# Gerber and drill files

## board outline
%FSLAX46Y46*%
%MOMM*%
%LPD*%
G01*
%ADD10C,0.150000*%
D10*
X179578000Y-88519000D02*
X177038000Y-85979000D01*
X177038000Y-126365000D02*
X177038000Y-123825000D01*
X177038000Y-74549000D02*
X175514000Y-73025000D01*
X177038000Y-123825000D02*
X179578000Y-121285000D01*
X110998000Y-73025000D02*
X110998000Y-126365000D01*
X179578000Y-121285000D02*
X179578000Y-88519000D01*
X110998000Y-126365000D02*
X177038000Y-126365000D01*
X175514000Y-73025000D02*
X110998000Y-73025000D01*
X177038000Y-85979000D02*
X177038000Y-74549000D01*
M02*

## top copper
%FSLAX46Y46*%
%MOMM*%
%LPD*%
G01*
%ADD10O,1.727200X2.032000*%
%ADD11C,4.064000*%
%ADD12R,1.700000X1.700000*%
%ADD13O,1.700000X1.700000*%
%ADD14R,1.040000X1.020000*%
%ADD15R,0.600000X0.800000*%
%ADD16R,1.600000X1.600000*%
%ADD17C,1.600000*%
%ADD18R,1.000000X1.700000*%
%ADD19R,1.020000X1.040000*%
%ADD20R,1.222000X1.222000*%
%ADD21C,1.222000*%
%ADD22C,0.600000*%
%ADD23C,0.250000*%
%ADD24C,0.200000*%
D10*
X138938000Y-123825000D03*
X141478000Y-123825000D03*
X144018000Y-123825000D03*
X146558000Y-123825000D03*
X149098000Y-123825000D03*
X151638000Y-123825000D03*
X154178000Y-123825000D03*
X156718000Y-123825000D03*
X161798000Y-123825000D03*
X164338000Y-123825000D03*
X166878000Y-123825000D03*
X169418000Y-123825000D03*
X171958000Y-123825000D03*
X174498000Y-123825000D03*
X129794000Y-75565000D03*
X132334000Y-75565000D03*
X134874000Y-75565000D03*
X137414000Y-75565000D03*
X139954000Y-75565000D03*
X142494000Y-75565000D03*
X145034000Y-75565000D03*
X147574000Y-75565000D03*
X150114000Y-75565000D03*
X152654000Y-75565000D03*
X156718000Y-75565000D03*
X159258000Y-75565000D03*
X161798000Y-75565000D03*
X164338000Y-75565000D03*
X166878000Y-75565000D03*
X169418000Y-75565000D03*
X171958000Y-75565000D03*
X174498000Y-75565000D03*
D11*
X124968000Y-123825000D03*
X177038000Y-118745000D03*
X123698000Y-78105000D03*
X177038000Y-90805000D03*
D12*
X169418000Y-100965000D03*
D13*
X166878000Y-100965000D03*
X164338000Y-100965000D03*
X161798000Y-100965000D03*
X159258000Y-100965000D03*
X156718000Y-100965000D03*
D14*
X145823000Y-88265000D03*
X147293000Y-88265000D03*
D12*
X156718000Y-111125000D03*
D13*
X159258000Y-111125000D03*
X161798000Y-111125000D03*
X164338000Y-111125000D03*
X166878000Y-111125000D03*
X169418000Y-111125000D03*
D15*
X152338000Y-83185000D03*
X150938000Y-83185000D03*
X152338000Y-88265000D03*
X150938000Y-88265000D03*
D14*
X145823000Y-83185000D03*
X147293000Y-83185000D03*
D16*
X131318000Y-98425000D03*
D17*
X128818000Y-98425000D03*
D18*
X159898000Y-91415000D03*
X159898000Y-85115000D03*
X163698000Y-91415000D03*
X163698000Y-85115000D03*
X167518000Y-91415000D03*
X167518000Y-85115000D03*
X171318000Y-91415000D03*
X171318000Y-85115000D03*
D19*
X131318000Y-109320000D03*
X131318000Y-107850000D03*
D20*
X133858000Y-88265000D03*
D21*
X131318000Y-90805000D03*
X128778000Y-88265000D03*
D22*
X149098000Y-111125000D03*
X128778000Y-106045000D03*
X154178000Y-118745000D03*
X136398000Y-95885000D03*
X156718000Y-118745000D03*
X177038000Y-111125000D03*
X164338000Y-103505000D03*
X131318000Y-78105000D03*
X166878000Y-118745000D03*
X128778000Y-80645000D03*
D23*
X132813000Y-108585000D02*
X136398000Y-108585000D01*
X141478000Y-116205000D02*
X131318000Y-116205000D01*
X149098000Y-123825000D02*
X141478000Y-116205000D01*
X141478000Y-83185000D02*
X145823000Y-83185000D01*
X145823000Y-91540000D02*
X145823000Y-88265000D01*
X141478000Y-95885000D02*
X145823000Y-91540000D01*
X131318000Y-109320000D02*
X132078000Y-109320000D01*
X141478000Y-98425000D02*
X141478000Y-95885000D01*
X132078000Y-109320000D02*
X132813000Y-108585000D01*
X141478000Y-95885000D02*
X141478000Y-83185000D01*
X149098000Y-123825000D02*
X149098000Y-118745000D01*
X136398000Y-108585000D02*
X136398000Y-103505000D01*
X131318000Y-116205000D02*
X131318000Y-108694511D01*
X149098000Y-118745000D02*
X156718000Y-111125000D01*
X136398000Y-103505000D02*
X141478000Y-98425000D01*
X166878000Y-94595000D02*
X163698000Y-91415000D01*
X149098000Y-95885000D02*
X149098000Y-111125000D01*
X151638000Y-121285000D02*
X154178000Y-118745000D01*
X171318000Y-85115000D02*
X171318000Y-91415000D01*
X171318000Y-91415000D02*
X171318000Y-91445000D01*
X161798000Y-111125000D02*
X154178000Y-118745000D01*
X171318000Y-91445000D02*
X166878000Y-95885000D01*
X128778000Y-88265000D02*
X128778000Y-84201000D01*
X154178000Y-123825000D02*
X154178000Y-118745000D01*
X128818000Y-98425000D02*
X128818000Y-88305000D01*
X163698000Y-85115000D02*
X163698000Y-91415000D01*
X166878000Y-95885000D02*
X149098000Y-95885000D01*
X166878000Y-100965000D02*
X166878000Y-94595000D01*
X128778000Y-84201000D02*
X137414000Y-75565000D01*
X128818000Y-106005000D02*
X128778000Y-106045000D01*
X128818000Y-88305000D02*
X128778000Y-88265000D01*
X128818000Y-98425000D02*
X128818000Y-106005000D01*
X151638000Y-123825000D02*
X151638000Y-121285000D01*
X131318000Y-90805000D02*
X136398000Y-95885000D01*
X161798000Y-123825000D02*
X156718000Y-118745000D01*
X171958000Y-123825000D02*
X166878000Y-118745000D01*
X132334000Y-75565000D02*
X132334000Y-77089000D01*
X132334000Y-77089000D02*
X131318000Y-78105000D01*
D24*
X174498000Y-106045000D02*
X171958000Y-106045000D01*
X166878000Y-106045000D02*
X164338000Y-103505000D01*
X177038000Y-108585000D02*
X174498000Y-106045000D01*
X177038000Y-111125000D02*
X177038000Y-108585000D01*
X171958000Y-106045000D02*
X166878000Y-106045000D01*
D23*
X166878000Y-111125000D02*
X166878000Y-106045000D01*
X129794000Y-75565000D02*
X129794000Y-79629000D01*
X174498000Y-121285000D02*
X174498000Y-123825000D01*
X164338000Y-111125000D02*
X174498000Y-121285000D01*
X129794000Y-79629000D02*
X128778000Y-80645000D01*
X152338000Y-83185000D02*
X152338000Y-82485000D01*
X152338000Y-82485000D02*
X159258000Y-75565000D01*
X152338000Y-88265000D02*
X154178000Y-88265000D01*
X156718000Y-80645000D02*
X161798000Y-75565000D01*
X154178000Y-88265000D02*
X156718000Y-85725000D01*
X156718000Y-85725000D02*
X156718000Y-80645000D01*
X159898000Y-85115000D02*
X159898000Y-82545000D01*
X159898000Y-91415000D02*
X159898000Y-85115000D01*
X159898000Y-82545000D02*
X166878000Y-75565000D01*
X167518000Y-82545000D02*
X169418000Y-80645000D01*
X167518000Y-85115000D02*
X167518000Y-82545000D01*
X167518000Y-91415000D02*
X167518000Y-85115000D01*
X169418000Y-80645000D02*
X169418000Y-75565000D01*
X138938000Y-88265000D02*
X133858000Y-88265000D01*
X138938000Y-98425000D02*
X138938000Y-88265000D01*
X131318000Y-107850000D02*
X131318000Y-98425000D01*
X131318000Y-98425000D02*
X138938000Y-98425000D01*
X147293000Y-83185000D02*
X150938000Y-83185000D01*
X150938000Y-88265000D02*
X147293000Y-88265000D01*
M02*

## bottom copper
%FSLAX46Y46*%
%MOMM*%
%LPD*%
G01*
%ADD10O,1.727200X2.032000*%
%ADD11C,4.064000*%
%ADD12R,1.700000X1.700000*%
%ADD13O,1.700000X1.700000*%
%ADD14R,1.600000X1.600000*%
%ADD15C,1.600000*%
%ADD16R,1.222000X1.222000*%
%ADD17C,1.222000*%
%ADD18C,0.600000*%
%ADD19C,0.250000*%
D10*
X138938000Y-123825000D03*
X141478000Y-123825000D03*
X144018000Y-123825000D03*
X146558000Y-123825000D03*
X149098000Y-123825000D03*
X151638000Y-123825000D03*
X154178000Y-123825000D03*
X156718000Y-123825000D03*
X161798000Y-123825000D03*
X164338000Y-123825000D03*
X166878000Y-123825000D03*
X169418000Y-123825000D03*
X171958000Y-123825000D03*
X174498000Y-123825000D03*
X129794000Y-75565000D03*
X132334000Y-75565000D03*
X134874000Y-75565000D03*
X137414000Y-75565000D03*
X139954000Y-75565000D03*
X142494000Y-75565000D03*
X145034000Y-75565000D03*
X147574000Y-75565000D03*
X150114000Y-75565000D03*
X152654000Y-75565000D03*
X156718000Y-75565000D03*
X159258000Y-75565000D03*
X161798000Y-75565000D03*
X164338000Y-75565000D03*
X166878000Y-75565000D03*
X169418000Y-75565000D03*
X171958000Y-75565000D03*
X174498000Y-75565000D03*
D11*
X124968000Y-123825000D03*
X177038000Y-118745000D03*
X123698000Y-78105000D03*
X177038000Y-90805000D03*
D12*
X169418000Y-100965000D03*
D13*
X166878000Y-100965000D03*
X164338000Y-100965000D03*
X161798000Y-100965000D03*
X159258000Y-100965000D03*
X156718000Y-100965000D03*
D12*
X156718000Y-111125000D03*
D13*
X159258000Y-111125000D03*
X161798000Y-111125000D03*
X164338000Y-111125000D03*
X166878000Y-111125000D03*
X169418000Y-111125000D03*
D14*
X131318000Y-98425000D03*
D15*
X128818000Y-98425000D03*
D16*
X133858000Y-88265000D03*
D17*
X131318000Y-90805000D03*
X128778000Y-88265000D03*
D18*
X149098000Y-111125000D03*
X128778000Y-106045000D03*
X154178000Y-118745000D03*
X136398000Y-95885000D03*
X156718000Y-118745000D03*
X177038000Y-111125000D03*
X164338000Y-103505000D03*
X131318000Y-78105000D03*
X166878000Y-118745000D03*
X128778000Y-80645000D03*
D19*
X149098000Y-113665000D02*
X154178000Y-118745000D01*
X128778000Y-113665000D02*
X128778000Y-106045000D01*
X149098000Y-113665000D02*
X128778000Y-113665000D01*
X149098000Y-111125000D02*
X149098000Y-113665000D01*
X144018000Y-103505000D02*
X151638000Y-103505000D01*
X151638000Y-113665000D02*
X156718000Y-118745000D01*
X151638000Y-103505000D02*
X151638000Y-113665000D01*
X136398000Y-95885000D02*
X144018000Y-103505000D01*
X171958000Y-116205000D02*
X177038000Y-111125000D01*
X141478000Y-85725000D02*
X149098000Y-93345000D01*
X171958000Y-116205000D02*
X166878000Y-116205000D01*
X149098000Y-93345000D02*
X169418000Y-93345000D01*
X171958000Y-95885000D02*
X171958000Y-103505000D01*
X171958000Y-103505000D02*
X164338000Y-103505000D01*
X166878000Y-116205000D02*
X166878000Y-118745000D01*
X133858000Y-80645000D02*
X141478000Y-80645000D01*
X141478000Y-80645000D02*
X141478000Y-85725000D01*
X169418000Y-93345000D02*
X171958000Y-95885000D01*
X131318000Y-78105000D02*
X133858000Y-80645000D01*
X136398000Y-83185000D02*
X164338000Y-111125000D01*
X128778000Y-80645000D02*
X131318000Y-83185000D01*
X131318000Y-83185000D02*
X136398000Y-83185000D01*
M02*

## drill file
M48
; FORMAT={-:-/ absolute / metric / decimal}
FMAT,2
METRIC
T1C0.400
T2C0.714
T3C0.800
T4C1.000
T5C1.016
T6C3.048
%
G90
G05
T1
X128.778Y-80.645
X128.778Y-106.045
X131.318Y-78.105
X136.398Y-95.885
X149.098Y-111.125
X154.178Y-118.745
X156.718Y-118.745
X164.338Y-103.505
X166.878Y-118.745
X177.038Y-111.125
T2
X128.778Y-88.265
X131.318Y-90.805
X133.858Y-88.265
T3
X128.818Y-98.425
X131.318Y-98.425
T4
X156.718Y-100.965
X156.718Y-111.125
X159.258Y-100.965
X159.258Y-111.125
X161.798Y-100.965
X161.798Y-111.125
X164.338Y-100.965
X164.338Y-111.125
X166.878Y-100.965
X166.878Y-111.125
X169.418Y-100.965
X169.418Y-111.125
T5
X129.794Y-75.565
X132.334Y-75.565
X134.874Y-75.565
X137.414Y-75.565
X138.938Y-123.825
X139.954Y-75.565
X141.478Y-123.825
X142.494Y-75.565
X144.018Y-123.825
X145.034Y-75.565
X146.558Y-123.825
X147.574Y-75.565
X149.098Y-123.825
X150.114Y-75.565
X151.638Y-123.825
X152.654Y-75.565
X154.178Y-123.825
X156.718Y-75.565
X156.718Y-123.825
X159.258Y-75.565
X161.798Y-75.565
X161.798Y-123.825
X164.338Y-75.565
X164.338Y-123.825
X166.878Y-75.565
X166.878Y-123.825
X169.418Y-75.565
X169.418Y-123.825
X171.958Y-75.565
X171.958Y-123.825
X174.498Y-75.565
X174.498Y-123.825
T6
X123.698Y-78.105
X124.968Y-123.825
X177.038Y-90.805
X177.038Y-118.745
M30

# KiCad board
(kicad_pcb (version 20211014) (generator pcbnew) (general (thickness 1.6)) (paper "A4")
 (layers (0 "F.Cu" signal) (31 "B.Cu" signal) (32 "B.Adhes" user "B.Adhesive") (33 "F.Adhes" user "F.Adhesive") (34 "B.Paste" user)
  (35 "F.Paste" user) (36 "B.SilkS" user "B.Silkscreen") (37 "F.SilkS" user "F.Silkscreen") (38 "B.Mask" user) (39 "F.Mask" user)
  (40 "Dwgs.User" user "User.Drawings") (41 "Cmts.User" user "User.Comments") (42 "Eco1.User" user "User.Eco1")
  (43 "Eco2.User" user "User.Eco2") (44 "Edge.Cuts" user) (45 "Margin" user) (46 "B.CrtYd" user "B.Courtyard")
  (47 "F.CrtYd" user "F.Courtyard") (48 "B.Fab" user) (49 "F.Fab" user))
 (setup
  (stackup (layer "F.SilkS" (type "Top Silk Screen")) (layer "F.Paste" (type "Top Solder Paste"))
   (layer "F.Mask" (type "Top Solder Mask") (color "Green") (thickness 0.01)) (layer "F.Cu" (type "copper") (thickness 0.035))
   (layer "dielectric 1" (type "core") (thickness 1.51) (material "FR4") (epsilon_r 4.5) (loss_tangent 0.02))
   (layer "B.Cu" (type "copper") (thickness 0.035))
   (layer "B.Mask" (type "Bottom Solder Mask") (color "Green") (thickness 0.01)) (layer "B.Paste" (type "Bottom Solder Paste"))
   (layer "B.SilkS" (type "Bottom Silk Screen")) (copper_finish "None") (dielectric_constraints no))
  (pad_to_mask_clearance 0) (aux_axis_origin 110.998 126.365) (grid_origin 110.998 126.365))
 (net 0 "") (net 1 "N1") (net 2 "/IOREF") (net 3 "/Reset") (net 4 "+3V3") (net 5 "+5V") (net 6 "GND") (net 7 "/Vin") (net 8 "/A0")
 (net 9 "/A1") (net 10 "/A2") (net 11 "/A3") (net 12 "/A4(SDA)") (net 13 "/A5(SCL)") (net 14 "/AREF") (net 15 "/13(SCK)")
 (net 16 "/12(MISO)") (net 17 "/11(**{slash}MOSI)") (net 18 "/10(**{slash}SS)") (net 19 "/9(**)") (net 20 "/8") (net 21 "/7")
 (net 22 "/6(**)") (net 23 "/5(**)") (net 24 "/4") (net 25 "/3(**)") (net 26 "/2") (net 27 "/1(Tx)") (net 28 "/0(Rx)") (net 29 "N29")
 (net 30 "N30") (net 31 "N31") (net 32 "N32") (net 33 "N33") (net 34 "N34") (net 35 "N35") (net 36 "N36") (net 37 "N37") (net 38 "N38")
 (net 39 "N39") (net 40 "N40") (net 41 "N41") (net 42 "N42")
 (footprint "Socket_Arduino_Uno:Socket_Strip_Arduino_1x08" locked (layer "F.Cu") (at 138.938 123.825)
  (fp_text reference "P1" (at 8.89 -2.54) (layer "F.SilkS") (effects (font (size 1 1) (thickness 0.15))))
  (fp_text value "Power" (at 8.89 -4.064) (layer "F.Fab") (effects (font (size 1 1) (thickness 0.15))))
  (pad "1" thru_hole oval locked (at 0 0) (size 1.7272 2.032) (drill 1.016) (layers *.Cu *.Mask "F.SilkS") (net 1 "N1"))
  (pad "2" thru_hole oval locked (at 2.54 0) (size 1.7272 2.032) (drill 1.016) (layers *.Cu *.Mask "F.SilkS") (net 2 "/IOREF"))
  (pad "3" thru_hole oval locked (at 5.08 0) (size 1.7272 2.032) (drill 1.016) (layers *.Cu *.Mask "F.SilkS") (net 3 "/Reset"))
  (pad "4" thru_hole oval locked (at 7.62 0) (size 1.7272 2.032) (drill 1.016) (layers *.Cu *.Mask "F.SilkS") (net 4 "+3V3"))
  (pad "5" thru_hole oval locked (at 10.16 0) (size 1.7272 2.032) (drill 1.016) (layers *.Cu *.Mask "F.SilkS") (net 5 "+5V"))
  (pad "6" thru_hole oval locked (at 12.7 0) (size 1.7272 2.032) (drill 1.016) (layers *.Cu *.Mask "F.SilkS") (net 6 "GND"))
  (pad "7" thru_hole oval locked (at 15.24 0) (size 1.7272 2.032) (drill 1.016) (layers *.Cu *.Mask "F.SilkS") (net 6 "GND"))
  (pad "8" thru_hole oval locked (at 17.78 0) (size 1.7272 2.032) (drill 1.016) (layers *.Cu *.Mask "F.SilkS") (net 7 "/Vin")))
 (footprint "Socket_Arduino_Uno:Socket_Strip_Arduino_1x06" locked (layer "F.Cu") (at 161.798 123.825)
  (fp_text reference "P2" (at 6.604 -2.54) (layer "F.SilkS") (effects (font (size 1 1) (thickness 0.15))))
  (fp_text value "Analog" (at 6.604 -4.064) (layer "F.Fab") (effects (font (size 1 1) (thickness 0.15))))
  (pad "1" thru_hole oval locked (at 0 0) (size 1.7272 2.032) (drill 1.016) (layers *.Cu *.Mask "F.SilkS") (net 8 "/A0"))
  (pad "2" thru_hole oval locked (at 2.54 0) (size 1.7272 2.032) (drill 1.016) (layers *.Cu *.Mask "F.SilkS") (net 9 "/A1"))
  (pad "3" thru_hole oval locked (at 5.08 0) (size 1.7272 2.032) (drill 1.016) (layers *.Cu *.Mask "F.SilkS") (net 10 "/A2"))
  (pad "4" thru_hole oval locked (at 7.62 0) (size 1.7272 2.032) (drill 1.016) (layers *.Cu *.Mask "F.SilkS") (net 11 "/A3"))
  (pad "5" thru_hole oval locked (at 10.16 0) (size 1.7272 2.032) (drill 1.016) (layers *.Cu *.Mask "F.SilkS") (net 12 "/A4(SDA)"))
  (pad "6" thru_hole oval locked (at 12.7 0) (size 1.7272 2.032) (drill 1.016) (layers *.Cu *.Mask "F.SilkS") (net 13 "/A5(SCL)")))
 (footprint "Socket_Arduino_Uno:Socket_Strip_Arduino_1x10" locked (layer "F.Cu") (at 129.794 75.565)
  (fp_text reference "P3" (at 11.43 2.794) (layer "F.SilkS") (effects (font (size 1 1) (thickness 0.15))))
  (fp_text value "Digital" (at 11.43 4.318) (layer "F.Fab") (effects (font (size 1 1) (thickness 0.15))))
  (pad "1" thru_hole oval locked (at 0 0) (size 1.7272 2.032) (drill 1.016) (layers *.Cu *.Mask "F.SilkS") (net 13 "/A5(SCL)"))
  (pad "2" thru_hole oval locked (at 2.54 0) (size 1.7272 2.032) (drill 1.016) (layers *.Cu *.Mask "F.SilkS") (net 12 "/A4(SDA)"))
  (pad "3" thru_hole oval locked (at 5.08 0) (size 1.7272 2.032) (drill 1.016) (layers *.Cu *.Mask "F.SilkS") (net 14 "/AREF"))
  (pad "4" thru_hole oval locked (at 7.62 0) (size 1.7272 2.032) (drill 1.016) (layers *.Cu *.Mask "F.SilkS") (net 6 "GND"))
  (pad "5" thru_hole oval locked (at 10.16 0) (size 1.7272 2.032) (drill 1.016) (layers *.Cu *.Mask "F.SilkS") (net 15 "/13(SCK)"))
  (pad "6" thru_hole oval locked (at 12.7 0) (size 1.7272 2.032) (drill 1.016) (layers *.Cu *.Mask "F.SilkS") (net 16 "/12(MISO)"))
  (pad "7" thru_hole oval locked (at 15.24 0) (size 1.7272 2.032) (drill 1.016) (layers *.Cu *.Mask "F.SilkS") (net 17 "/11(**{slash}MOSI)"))
  (pad "8" thru_hole oval locked (at 17.78 0) (size 1.7272 2.032) (drill 1.016) (layers *.Cu *.Mask "F.SilkS") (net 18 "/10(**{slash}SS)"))
  (pad "9" thru_hole oval locked (at 20.32 0) (size 1.7272 2.032) (drill 1.016) (layers *.Cu *.Mask "F.SilkS") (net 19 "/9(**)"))
  (pad "10" thru_hole oval locked (at 22.86 0) (size 1.7272 2.032) (drill 1.016) (layers *.Cu *.Mask "F.SilkS") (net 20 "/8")))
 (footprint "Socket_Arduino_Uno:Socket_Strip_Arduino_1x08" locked (layer "F.Cu") (at 156.718 75.565)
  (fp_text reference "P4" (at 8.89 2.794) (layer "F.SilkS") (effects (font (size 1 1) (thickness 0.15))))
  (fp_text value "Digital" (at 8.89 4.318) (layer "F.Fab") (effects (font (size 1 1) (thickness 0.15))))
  (pad "1" thru_hole oval locked (at 0 0) (size 1.7272 2.032) (drill 1.016) (layers *.Cu *.Mask "F.SilkS") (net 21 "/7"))
  (pad "2" thru_hole oval locked (at 2.54 0) (size 1.7272 2.032) (drill 1.016) (layers *.Cu *.Mask "F.SilkS") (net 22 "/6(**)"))
  (pad "3" thru_hole oval locked (at 5.08 0) (size 1.7272 2.032) (drill 1.016) (layers *.Cu *.Mask "F.SilkS") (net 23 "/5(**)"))
  (pad "4" thru_hole oval locked (at 7.62 0) (size 1.7272 2.032) (drill 1.016) (layers *.Cu *.Mask "F.SilkS") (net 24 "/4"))
  (pad "5" thru_hole oval locked (at 10.16 0) (size 1.7272 2.032) (drill 1.016) (layers *.Cu *.Mask "F.SilkS") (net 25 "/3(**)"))
  (pad "6" thru_hole oval locked (at 12.7 0) (size 1.7272 2.032) (drill 1.016) (layers *.Cu *.Mask "F.SilkS") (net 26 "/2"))
  (pad "7" thru_hole oval locked (at 15.24 0) (size 1.7272 2.032) (drill 1.016) (layers *.Cu *.Mask "F.SilkS") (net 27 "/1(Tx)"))
  (pad "8" thru_hole oval locked (at 17.78 0) (size 1.7272 2.032) (drill 1.016) (layers *.Cu *.Mask "F.SilkS") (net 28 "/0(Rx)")))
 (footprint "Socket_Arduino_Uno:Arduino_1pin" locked (layer "F.Cu") (at 124.968 123.825)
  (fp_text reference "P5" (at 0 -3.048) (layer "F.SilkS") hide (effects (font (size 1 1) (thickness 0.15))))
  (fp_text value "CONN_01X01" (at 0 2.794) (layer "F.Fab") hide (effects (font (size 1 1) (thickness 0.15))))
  (pad "1" thru_hole circle locked (at 0 0) (size 4.064 4.064) (drill 3.048) (layers *.Cu *.Mask "F.SilkS") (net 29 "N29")))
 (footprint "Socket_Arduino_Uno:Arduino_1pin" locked (layer "F.Cu") (at 177.038 118.745)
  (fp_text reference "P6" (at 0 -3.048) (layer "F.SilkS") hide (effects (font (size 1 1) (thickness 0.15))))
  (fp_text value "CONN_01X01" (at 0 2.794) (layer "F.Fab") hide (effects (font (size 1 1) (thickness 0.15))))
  (pad "1" thru_hole circle locked (at 0 0) (size 4.064 4.064) (drill 3.048) (layers *.Cu *.Mask "F.SilkS") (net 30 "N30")))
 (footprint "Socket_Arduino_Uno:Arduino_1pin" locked (layer "F.Cu") (at 123.698 78.105)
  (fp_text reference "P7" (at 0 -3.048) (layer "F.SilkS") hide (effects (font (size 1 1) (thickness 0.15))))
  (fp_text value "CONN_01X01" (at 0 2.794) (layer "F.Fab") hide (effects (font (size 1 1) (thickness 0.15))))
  (pad "1" thru_hole circle locked (at 0 0) (size 4.064 4.064) (drill 3.048) (layers *.Cu *.Mask "F.SilkS") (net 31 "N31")))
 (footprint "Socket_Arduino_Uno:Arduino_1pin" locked (layer "F.Cu") (at 177.038 90.805)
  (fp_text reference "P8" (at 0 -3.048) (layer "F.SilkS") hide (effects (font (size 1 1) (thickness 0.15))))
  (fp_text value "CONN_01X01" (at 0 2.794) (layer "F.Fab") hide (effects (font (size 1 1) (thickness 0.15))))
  (pad "1" thru_hole circle locked (at 0 0) (size 4.064 4.064) (drill 3.048) (layers *.Cu *.Mask "F.SilkS") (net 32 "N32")))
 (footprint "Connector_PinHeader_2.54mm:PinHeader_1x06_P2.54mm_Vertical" (layer "F.Cu") (at 169.418 100.965 -90)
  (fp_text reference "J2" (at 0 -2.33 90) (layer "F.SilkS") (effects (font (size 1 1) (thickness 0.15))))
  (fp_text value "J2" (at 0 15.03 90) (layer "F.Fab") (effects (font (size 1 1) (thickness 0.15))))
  (pad "1" thru_hole rect (at 0 0 270) (size 1.7 1.7) (drill 1) (layers *.Cu *.Mask) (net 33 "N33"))
  (pad "2" thru_hole oval (at 0 2.54 270) (size 1.7 1.7) (drill 1) (layers *.Cu *.Mask) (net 6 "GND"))
  (pad "3" thru_hole oval (at 0 5.08 270) (size 1.7 1.7) (drill 1) (layers *.Cu *.Mask) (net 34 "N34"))
  (pad "4" thru_hole oval (at 0 7.62 270) (size 1.7 1.7) (drill 1) (layers *.Cu *.Mask) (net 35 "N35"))
  (pad "5" thru_hole oval (at 0 10.16 270) (size 1.7 1.7) (drill 1) (layers *.Cu *.Mask) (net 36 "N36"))
  (pad "6" thru_hole oval (at 0 12.7 270) (size 1.7 1.7) (drill 1) (layers *.Cu *.Mask) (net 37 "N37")))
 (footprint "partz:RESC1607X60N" (layer "F.Cu") (at 146.558 88.265)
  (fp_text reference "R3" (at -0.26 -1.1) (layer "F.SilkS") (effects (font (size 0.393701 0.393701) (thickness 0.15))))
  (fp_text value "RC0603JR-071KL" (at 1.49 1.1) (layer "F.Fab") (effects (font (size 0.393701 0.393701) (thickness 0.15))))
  (pad "1" smd rect locked (at -0.735 0) (size 1.04 1.02) (layers "F.Cu" "F.Paste" "F.Mask") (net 5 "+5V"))
  (pad "2" smd rect locked (at 0.735 0) (size 1.04 1.02) (layers "F.Cu" "F.Paste" "F.Mask") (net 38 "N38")))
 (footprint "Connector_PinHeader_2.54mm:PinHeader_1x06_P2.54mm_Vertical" (layer "F.Cu") (at 156.718 111.125 90)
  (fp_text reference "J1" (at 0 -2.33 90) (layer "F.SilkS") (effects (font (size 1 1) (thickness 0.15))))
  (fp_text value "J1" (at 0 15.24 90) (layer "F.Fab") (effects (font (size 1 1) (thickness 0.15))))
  (pad "1" thru_hole rect (at 0 0 90) (size 1.7 1.7) (drill 1) (layers *.Cu *.Mask) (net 5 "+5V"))
  (pad "2" thru_hole oval (at 0 2.54 90) (size 1.7 1.7) (drill 1) (layers *.Cu *.Mask) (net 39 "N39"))
  (pad "3" thru_hole oval (at 0 5.08 90) (size 1.7 1.7) (drill 1) (layers *.Cu *.Mask) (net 6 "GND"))
  (pad "4" thru_hole oval (at 0 7.62 90) (size 1.7 1.7) (drill 1) (layers *.Cu *.Mask) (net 13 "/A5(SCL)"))
  (pad "5" thru_hole oval (at 0 10.16 90) (size 1.7 1.7) (drill 1) (layers *.Cu *.Mask) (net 12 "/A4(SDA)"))
  (pad "6" thru_hole oval (at 0 12.7 90) (size 1.7 1.7) (drill 1) (layers *.Cu *.Mask) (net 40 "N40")))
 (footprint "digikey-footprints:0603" (layer "F.Cu") (at 151.638 83.185 180)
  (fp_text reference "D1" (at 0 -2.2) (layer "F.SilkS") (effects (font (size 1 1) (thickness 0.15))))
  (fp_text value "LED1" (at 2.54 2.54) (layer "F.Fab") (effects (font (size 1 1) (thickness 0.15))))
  (pad "1" smd rect locked (at -0.7 0 180) (size 0.6 0.8) (layers "F.Cu" "F.Paste" "F.Mask") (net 22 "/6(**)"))
  (pad "2" smd rect locked (at 0.7 0 180) (size 0.6 0.8) (layers "F.Cu" "F.Paste" "F.Mask") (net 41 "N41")))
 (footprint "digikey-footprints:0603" (layer "F.Cu") (at 151.638 88.265 180)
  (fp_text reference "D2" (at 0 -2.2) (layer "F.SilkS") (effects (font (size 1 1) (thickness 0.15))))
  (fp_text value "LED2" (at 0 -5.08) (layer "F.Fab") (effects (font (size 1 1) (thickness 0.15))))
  (pad "1" smd rect locked (at -0.7 0 180) (size 0.6 0.8) (layers "F.Cu" "F.Paste" "F.Mask") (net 23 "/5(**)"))
  (pad "2" smd rect locked (at 0.7 0 180) (size 0.6 0.8) (layers "F.Cu" "F.Paste" "F.Mask") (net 38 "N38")))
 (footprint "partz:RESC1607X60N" (layer "F.Cu") (at 146.558 83.185)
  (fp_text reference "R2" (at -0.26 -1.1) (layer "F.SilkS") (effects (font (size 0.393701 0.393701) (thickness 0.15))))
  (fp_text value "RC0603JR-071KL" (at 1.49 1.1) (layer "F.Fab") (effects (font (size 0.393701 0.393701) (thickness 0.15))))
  (pad "1" smd rect locked (at -0.735 0) (size 1.04 1.02) (layers "F.Cu" "F.Paste" "F.Mask") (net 5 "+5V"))
  (pad "2" smd rect locked (at 0.735 0) (size 1.04 1.02) (layers "F.Cu" "F.Paste" "F.Mask") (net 41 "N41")))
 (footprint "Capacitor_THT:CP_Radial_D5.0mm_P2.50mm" (layer "F.Cu") (at 131.318 98.425 180)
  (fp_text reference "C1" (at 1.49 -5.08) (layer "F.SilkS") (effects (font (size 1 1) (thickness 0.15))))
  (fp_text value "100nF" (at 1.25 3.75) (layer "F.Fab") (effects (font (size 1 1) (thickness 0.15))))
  (pad "1" thru_hole rect (at 0 0 180) (size 1.6 1.6) (drill 0.8) (layers *.Cu *.Mask) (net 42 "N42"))
  (pad "2" thru_hole circle (at 2.5 0 180) (size 1.6 1.6) (drill 0.8) (layers *.Cu *.Mask) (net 6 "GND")))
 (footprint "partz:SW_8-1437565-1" (layer "F.Cu") (at 161.798 88.265 90)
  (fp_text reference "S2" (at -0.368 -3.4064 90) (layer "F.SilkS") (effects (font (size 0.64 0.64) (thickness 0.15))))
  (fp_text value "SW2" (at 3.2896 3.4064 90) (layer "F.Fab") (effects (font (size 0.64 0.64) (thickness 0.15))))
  (pad "1" smd rect locked (at -3.15 -1.9 90) (size 1.7 1) (layers "F.Cu" "F.Paste" "F.Mask") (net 25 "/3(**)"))
  (pad "2" smd rect locked (at 3.15 -1.9 90) (size 1.7 1) (layers "F.Cu" "F.Paste" "F.Mask") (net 25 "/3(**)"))
  (pad "3" smd rect locked (at -3.15 1.9 90) (size 1.7 1) (layers "F.Cu" "F.Paste" "F.Mask") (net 6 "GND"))
  (pad "4" smd rect locked (at 3.15 1.9 90) (size 1.7 1) (layers "F.Cu" "F.Paste" "F.Mask") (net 6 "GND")))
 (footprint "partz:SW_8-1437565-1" (layer "F.Cu") (at 169.418 88.265 90)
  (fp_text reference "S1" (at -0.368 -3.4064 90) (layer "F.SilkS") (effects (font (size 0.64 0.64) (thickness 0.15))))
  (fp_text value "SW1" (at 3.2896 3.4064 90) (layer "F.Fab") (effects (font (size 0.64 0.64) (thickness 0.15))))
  (pad "1" smd rect locked (at -3.15 -1.9 90) (size 1.7 1) (layers "F.Cu" "F.Paste" "F.Mask") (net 26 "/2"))
  (pad "2" smd rect locked (at 3.15 -1.9 90) (size 1.7 1) (layers "F.Cu" "F.Paste" "F.Mask") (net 26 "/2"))
  (pad "3" smd rect locked (at -3.15 1.9 90) (size 1.7 1) (layers "F.Cu" "F.Paste" "F.Mask") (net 6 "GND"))
  (pad "4" smd rect locked (at 3.15 1.9 90) (size 1.7 1) (layers "F.Cu" "F.Paste" "F.Mask") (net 6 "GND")))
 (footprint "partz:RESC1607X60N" (layer "F.Cu") (at 131.318 108.585 90)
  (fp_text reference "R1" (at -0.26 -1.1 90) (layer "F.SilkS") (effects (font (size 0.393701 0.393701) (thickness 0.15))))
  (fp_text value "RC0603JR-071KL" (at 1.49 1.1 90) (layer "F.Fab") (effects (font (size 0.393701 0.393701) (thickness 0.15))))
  (pad "1" smd rect locked (at -0.735 0 90) (size 1.04 1.02) (layers "F.Cu" "F.Paste" "F.Mask") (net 5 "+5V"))
  (pad "2" smd rect locked (at 0.735 0 90) (size 1.04 1.02) (layers "F.Cu" "F.Paste" "F.Mask") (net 42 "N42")))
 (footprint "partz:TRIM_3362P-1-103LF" (layer "F.Cu") (at 131.318 88.265 180)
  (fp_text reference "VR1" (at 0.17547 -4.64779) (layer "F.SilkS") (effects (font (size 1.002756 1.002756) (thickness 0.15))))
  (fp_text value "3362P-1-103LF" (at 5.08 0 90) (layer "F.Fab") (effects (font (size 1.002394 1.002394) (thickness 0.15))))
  (pad "1" thru_hole rect locked (at -2.54 0 180) (size 1.222 1.222) (drill 0.714) (layers *.Cu *.Mask) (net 42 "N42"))
  (pad "2" thru_hole circle locked (at 0 -2.54 180) (size 1.222 1.222) (drill 0.714) (layers *.Cu *.Mask) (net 8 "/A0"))
  (pad "3" thru_hole circle locked (at 2.54 0 180) (size 1.222 1.222) (drill 0.714) (layers *.Cu *.Mask) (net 6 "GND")))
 (gr_line (start 179.578 88.519) (end 177.038 85.979) (layer "Edge.Cuts") (width 0.15))
 (gr_line (start 177.038 126.365) (end 177.038 123.825) (layer "Edge.Cuts") (width 0.15))
 (gr_line (start 177.038 74.549) (end 175.514 73.025) (layer "Edge.Cuts") (width 0.15))
 (gr_line (start 177.038 123.825) (end 179.578 121.285) (layer "Edge.Cuts") (width 0.15))
 (gr_line (start 110.998 73.025) (end 110.998 126.365) (layer "Edge.Cuts") (width 0.15))
 (gr_line (start 179.578 121.285) (end 179.578 88.519) (layer "Edge.Cuts") (width 0.15))
 (gr_line (start 110.998 126.365) (end 177.038 126.365) (layer "Edge.Cuts") (width 0.15))
 (gr_line (start 175.514 73.025) (end 110.998 73.025) (layer "Edge.Cuts") (width 0.15))
 (gr_line (start 177.038 85.979) (end 177.038 74.549) (layer "Edge.Cuts") (width 0.15))
 (segment (start 132.813 108.585) (end 136.398 108.585) (width 0.25) (layer "F.Cu") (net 5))
 (segment (start 141.478 116.205) (end 131.318 116.205) (width 0.25) (layer "F.Cu") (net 5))
 (segment (start 149.098 123.825) (end 141.478 116.205) (width 0.25) (layer "F.Cu") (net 5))
 (segment (start 141.478 83.185) (end 145.823 83.185) (width 0.25) (layer "F.Cu") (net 5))
 (segment (start 145.823 91.54) (end 145.823 88.265) (width 0.25) (layer "F.Cu") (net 5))
 (segment (start 141.478 95.885) (end 145.823 91.54) (width 0.25) (layer "F.Cu") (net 5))
 (segment (start 131.318 109.32) (end 132.078 109.32) (width 0.25) (layer "F.Cu") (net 5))
 (segment (start 141.478 98.425) (end 141.478 95.885) (width 0.25) (layer "F.Cu") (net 5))
 (segment (start 132.078 109.32) (end 132.813 108.585) (width 0.25) (layer "F.Cu") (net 5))
 (segment (start 141.478 95.885) (end 141.478 83.185) (width 0.25) (layer "F.Cu") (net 5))
 (segment (start 149.098 123.825) (end 149.098 118.745) (width 0.25) (layer "F.Cu") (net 5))
 (segment (start 136.398 108.585) (end 136.398 103.505) (width 0.25) (layer "F.Cu") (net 5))
 (segment (start 131.318 116.205) (end 131.318 108.694511) (width 0.25) (layer "F.Cu") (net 5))
 (segment (start 149.098 118.745) (end 156.718 111.125) (width 0.25) (layer "F.Cu") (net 5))
 (segment (start 136.398 103.505) (end 141.478 98.425) (width 0.25) (layer "F.Cu") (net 5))
 (segment (start 166.878 94.595) (end 163.698 91.415) (width 0.25) (layer "F.Cu") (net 6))
 (segment (start 149.098 95.885) (end 149.098 111.125) (width 0.25) (layer "F.Cu") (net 6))
 (segment (start 151.638 121.285) (end 154.178 118.745) (width 0.25) (layer "F.Cu") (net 6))
 (segment (start 171.318 85.115) (end 171.318 91.415) (width 0.25) (layer "F.Cu") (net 6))
 (segment (start 171.318 91.415) (end 171.318 91.445) (width 0.25) (layer "F.Cu") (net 6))
 (segment (start 161.798 111.125) (end 154.178 118.745) (width 0.25) (layer "F.Cu") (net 6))
 (segment (start 171.318 91.445) (end 166.878 95.885) (width 0.25) (layer "F.Cu") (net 6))
 (segment (start 128.778 88.265) (end 128.778 84.201) (width 0.25) (layer "F.Cu") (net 6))
 (segment (start 154.178 123.825) (end 154.178 118.745) (width 0.25) (layer "F.Cu") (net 6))
 (segment (start 128.818 98.425) (end 128.818 88.305) (width 0.25) (layer "F.Cu") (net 6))
 (segment (start 163.698 85.115) (end 163.698 91.415) (width 0.25) (layer "F.Cu") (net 6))
 (segment (start 166.878 95.885) (end 149.098 95.885) (width 0.25) (layer "F.Cu") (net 6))
 (segment (start 166.878 100.965) (end 166.878 94.595) (width 0.25) (layer "F.Cu") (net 6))
 (segment (start 128.778 84.201) (end 137.414 75.565) (width 0.25) (layer "F.Cu") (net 6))
 (segment (start 128.818 106.005) (end 128.778 106.045) (width 0.25) (layer "F.Cu") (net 6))
 (segment (start 128.818 88.305) (end 128.778 88.265) (width 0.25) (layer "F.Cu") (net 6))
 (segment (start 128.818 98.425) (end 128.818 106.005) (width 0.25) (layer "F.Cu") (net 6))
 (segment (start 151.638 123.825) (end 151.638 121.285) (width 0.25) (layer "F.Cu") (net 6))
 (via (at 149.098 111.125) (size 0.6) (drill 0.4) (layers "F.Cu" "B.Cu") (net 6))
 (via (at 128.778 106.045) (size 0.6) (drill 0.4) (layers "F.Cu" "B.Cu") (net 6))
 (via (at 154.178 118.745) (size 0.6) (drill 0.4) (layers "F.Cu" "B.Cu") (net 6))
 (segment (start 149.098 113.665) (end 154.178 118.745) (width 0.25) (layer "B.Cu") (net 6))
 (segment (start 128.778 113.665) (end 128.778 106.045) (width 0.25) (layer "B.Cu") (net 6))
 (segment (start 149.098 113.665) (end 128.778 113.665) (width 0.25) (layer "B.Cu") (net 6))
 (segment (start 149.098 111.125) (end 149.098 113.665) (width 0.25) (layer "B.Cu") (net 6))
 (segment (start 131.318 90.805) (end 136.398 95.885) (width 0.25) (layer "F.Cu") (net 8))
 (segment (start 161.798 123.825) (end 156.718 118.745) (width 0.25) (layer "F.Cu") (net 8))
 (via (at 136.398 95.885) (size 0.6) (drill 0.4) (layers "F.Cu" "B.Cu") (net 8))
 (via (at 156.718 118.745) (size 0.6) (drill 0.4) (layers "F.Cu" "B.Cu") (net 8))
 (segment (start 144.018 103.505) (end 151.638 103.505) (width 0.25) (layer "B.Cu") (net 8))
 (segment (start 151.638 113.665) (end 156.718 118.745) (width 0.25) (layer "B.Cu") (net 8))
 (segment (start 151.638 103.505) (end 151.638 113.665) (width 0.25) (layer "B.Cu") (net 8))
 (segment (start 136.398 95.885) (end 144.018 103.505) (width 0.25) (layer "B.Cu") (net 8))
 (segment (start 171.958 123.825) (end 166.878 118.745) (width 0.25) (layer "F.Cu") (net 12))
 (segment (start 132.334 75.565) (end 132.334 77.089) (width 0.25) (layer "F.Cu") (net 12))
 (segment (start 132.334 77.089) (end 131.318 78.105) (width 0.25) (layer "F.Cu") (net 12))
 (segment (start 174.498 106.045) (end 171.958 106.045) (width 0.2) (layer "F.Cu") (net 12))
 (segment (start 166.878 106.045) (end 164.338 103.505) (width 0.2) (layer "F.Cu") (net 12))
 (segment (start 177.038 108.585) (end 174.498 106.045) (width 0.2) (layer "F.Cu") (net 12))
 (segment (start 177.038 111.125) (end 177.038 108.585) (width 0.2) (layer "F.Cu") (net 12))
 (segment (start 171.958 106.045) (end 166.878 106.045) (width 0.2) (layer "F.Cu") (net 12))
 (segment (start 166.878 111.125) (end 166.878 106.045) (width 0.25) (layer "F.Cu") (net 12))
 (via (at 177.038 111.125) (size 0.6) (drill 0.4) (layers "F.Cu" "B.Cu") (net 12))
 (via (at 164.338 103.505) (size 0.6) (drill 0.4) (layers "F.Cu" "B.Cu") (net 12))
 (via (at 131.318 78.105) (size 0.6) (drill 0.4) (layers "F.Cu" "B.Cu") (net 12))
 (via (at 166.878 118.745) (size 0.6) (drill 0.4) (layers "F.Cu" "B.Cu") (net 12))
 (segment (start 171.958 116.205) (end 177.038 111.125) (width 0.25) (layer "B.Cu") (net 12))
 (segment (start 141.478 85.725) (end 149.098 93.345) (width 0.25) (layer "B.Cu") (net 12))
 (segment (start 171.958 116.205) (end 166.878 116.205) (width 0.25) (layer "B.Cu") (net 12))
 (segment (start 149.098 93.345) (end 169.418 93.345) (width 0.25) (layer "B.Cu") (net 12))
 (segment (start 171.958 95.885) (end 171.958 103.505) (width 0.25) (layer "B.Cu") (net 12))
 (segment (start 171.958 103.505) (end 164.338 103.505) (width 0.25) (layer "B.Cu") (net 12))
 (segment (start 166.878 116.205) (end 166.878 118.745) (width 0.25) (layer "B.Cu") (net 12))
 (segment (start 133.858 80.645) (end 141.478 80.645) (width 0.25) (layer "B.Cu") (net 12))
 (segment (start 141.478 80.645) (end 141.478 85.725) (width 0.25) (layer "B.Cu") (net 12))
 (segment (start 169.418 93.345) (end 171.958 95.885) (width 0.25) (layer "B.Cu") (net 12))
 (segment (start 131.318 78.105) (end 133.858 80.645) (width 0.25) (layer "B.Cu") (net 12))
 (segment (start 129.794 75.565) (end 129.794 79.629) (width 0.25) (layer "F.Cu") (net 13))
 (segment (start 174.498 121.285) (end 174.498 123.825) (width 0.25) (layer "F.Cu") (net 13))
 (segment (start 164.338 111.125) (end 174.498 121.285) (width 0.25) (layer "F.Cu") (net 13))
 (segment (start 129.794 79.629) (end 128.778 80.645) (width 0.25) (layer "F.Cu") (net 13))
 (via (at 128.778 80.645) (size 0.6) (drill 0.4) (layers "F.Cu" "B.Cu") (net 13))
 (segment (start 136.398 83.185) (end 164.338 111.125) (width 0.25) (layer "B.Cu") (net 13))
 (segment (start 128.778 80.645) (end 131.318 83.185) (width 0.25) (layer "B.Cu") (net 13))
 (segment (start 131.318 83.185) (end 136.398 83.185) (width 0.25) (layer "B.Cu") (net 13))
 (segment (start 152.338 83.185) (end 152.338 82.485) (width 0.25) (layer "F.Cu") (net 22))
 (segment (start 152.338 82.485) (end 159.258 75.565) (width 0.25) (layer "F.Cu") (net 22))
 (segment (start 152.338 88.265) (end 154.178 88.265) (width 0.25) (layer "F.Cu") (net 23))
 (segment (start 156.718 80.645) (end 161.798 75.565) (width 0.25) (layer "F.Cu") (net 23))
 (segment (start 154.178 88.265) (end 156.718 85.725) (width 0.25) (layer "F.Cu") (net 23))
 (segment (start 156.718 85.725) (end 156.718 80.645) (width 0.25) (layer "F.Cu") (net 23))
 (segment (start 159.898 85.115) (end 159.898 82.545) (width 0.25) (layer "F.Cu") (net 25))
 (segment (start 159.898 91.415) (end 159.898 85.115) (width 0.25) (layer "F.Cu") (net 25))
 (segment (start 159.898 82.545) (end 166.878 75.565) (width 0.25) (layer "F.Cu") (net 25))
 (segment (start 167.518 82.545) (end 169.418 80.645) (width 0.25) (layer "F.Cu") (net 26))
 (segment (start 167.518 85.115) (end 167.518 82.545) (width 0.25) (layer "F.Cu") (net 26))
 (segment (start 167.518 91.415) (end 167.518 85.115) (width 0.25) (layer "F.Cu") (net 26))
 (segment (start 169.418 80.645) (end 169.418 75.565) (width 0.25) (layer "F.Cu") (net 26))
 (segment (start 138.938 88.265) (end 133.858 88.265) (width 0.25) (layer "F.Cu") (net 42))
 (segment (start 138.938 98.425) (end 138.938 88.265) (width 0.25) (layer "F.Cu") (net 42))
 (segment (start 131.318 107.85) (end 131.318 98.425) (width 0.25) (layer "F.Cu") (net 42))
 (segment (start 131.318 98.425) (end 138.938 98.425) (width 0.25) (layer "F.Cu") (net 42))
 (segment (start 147.293 83.185) (end 150.938 83.185) (width 0.25) (layer "F.Cu") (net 41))
 (segment (start 150.938 88.265) (end 147.293 88.265) (width 0.25) (layer "F.Cu") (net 38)))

